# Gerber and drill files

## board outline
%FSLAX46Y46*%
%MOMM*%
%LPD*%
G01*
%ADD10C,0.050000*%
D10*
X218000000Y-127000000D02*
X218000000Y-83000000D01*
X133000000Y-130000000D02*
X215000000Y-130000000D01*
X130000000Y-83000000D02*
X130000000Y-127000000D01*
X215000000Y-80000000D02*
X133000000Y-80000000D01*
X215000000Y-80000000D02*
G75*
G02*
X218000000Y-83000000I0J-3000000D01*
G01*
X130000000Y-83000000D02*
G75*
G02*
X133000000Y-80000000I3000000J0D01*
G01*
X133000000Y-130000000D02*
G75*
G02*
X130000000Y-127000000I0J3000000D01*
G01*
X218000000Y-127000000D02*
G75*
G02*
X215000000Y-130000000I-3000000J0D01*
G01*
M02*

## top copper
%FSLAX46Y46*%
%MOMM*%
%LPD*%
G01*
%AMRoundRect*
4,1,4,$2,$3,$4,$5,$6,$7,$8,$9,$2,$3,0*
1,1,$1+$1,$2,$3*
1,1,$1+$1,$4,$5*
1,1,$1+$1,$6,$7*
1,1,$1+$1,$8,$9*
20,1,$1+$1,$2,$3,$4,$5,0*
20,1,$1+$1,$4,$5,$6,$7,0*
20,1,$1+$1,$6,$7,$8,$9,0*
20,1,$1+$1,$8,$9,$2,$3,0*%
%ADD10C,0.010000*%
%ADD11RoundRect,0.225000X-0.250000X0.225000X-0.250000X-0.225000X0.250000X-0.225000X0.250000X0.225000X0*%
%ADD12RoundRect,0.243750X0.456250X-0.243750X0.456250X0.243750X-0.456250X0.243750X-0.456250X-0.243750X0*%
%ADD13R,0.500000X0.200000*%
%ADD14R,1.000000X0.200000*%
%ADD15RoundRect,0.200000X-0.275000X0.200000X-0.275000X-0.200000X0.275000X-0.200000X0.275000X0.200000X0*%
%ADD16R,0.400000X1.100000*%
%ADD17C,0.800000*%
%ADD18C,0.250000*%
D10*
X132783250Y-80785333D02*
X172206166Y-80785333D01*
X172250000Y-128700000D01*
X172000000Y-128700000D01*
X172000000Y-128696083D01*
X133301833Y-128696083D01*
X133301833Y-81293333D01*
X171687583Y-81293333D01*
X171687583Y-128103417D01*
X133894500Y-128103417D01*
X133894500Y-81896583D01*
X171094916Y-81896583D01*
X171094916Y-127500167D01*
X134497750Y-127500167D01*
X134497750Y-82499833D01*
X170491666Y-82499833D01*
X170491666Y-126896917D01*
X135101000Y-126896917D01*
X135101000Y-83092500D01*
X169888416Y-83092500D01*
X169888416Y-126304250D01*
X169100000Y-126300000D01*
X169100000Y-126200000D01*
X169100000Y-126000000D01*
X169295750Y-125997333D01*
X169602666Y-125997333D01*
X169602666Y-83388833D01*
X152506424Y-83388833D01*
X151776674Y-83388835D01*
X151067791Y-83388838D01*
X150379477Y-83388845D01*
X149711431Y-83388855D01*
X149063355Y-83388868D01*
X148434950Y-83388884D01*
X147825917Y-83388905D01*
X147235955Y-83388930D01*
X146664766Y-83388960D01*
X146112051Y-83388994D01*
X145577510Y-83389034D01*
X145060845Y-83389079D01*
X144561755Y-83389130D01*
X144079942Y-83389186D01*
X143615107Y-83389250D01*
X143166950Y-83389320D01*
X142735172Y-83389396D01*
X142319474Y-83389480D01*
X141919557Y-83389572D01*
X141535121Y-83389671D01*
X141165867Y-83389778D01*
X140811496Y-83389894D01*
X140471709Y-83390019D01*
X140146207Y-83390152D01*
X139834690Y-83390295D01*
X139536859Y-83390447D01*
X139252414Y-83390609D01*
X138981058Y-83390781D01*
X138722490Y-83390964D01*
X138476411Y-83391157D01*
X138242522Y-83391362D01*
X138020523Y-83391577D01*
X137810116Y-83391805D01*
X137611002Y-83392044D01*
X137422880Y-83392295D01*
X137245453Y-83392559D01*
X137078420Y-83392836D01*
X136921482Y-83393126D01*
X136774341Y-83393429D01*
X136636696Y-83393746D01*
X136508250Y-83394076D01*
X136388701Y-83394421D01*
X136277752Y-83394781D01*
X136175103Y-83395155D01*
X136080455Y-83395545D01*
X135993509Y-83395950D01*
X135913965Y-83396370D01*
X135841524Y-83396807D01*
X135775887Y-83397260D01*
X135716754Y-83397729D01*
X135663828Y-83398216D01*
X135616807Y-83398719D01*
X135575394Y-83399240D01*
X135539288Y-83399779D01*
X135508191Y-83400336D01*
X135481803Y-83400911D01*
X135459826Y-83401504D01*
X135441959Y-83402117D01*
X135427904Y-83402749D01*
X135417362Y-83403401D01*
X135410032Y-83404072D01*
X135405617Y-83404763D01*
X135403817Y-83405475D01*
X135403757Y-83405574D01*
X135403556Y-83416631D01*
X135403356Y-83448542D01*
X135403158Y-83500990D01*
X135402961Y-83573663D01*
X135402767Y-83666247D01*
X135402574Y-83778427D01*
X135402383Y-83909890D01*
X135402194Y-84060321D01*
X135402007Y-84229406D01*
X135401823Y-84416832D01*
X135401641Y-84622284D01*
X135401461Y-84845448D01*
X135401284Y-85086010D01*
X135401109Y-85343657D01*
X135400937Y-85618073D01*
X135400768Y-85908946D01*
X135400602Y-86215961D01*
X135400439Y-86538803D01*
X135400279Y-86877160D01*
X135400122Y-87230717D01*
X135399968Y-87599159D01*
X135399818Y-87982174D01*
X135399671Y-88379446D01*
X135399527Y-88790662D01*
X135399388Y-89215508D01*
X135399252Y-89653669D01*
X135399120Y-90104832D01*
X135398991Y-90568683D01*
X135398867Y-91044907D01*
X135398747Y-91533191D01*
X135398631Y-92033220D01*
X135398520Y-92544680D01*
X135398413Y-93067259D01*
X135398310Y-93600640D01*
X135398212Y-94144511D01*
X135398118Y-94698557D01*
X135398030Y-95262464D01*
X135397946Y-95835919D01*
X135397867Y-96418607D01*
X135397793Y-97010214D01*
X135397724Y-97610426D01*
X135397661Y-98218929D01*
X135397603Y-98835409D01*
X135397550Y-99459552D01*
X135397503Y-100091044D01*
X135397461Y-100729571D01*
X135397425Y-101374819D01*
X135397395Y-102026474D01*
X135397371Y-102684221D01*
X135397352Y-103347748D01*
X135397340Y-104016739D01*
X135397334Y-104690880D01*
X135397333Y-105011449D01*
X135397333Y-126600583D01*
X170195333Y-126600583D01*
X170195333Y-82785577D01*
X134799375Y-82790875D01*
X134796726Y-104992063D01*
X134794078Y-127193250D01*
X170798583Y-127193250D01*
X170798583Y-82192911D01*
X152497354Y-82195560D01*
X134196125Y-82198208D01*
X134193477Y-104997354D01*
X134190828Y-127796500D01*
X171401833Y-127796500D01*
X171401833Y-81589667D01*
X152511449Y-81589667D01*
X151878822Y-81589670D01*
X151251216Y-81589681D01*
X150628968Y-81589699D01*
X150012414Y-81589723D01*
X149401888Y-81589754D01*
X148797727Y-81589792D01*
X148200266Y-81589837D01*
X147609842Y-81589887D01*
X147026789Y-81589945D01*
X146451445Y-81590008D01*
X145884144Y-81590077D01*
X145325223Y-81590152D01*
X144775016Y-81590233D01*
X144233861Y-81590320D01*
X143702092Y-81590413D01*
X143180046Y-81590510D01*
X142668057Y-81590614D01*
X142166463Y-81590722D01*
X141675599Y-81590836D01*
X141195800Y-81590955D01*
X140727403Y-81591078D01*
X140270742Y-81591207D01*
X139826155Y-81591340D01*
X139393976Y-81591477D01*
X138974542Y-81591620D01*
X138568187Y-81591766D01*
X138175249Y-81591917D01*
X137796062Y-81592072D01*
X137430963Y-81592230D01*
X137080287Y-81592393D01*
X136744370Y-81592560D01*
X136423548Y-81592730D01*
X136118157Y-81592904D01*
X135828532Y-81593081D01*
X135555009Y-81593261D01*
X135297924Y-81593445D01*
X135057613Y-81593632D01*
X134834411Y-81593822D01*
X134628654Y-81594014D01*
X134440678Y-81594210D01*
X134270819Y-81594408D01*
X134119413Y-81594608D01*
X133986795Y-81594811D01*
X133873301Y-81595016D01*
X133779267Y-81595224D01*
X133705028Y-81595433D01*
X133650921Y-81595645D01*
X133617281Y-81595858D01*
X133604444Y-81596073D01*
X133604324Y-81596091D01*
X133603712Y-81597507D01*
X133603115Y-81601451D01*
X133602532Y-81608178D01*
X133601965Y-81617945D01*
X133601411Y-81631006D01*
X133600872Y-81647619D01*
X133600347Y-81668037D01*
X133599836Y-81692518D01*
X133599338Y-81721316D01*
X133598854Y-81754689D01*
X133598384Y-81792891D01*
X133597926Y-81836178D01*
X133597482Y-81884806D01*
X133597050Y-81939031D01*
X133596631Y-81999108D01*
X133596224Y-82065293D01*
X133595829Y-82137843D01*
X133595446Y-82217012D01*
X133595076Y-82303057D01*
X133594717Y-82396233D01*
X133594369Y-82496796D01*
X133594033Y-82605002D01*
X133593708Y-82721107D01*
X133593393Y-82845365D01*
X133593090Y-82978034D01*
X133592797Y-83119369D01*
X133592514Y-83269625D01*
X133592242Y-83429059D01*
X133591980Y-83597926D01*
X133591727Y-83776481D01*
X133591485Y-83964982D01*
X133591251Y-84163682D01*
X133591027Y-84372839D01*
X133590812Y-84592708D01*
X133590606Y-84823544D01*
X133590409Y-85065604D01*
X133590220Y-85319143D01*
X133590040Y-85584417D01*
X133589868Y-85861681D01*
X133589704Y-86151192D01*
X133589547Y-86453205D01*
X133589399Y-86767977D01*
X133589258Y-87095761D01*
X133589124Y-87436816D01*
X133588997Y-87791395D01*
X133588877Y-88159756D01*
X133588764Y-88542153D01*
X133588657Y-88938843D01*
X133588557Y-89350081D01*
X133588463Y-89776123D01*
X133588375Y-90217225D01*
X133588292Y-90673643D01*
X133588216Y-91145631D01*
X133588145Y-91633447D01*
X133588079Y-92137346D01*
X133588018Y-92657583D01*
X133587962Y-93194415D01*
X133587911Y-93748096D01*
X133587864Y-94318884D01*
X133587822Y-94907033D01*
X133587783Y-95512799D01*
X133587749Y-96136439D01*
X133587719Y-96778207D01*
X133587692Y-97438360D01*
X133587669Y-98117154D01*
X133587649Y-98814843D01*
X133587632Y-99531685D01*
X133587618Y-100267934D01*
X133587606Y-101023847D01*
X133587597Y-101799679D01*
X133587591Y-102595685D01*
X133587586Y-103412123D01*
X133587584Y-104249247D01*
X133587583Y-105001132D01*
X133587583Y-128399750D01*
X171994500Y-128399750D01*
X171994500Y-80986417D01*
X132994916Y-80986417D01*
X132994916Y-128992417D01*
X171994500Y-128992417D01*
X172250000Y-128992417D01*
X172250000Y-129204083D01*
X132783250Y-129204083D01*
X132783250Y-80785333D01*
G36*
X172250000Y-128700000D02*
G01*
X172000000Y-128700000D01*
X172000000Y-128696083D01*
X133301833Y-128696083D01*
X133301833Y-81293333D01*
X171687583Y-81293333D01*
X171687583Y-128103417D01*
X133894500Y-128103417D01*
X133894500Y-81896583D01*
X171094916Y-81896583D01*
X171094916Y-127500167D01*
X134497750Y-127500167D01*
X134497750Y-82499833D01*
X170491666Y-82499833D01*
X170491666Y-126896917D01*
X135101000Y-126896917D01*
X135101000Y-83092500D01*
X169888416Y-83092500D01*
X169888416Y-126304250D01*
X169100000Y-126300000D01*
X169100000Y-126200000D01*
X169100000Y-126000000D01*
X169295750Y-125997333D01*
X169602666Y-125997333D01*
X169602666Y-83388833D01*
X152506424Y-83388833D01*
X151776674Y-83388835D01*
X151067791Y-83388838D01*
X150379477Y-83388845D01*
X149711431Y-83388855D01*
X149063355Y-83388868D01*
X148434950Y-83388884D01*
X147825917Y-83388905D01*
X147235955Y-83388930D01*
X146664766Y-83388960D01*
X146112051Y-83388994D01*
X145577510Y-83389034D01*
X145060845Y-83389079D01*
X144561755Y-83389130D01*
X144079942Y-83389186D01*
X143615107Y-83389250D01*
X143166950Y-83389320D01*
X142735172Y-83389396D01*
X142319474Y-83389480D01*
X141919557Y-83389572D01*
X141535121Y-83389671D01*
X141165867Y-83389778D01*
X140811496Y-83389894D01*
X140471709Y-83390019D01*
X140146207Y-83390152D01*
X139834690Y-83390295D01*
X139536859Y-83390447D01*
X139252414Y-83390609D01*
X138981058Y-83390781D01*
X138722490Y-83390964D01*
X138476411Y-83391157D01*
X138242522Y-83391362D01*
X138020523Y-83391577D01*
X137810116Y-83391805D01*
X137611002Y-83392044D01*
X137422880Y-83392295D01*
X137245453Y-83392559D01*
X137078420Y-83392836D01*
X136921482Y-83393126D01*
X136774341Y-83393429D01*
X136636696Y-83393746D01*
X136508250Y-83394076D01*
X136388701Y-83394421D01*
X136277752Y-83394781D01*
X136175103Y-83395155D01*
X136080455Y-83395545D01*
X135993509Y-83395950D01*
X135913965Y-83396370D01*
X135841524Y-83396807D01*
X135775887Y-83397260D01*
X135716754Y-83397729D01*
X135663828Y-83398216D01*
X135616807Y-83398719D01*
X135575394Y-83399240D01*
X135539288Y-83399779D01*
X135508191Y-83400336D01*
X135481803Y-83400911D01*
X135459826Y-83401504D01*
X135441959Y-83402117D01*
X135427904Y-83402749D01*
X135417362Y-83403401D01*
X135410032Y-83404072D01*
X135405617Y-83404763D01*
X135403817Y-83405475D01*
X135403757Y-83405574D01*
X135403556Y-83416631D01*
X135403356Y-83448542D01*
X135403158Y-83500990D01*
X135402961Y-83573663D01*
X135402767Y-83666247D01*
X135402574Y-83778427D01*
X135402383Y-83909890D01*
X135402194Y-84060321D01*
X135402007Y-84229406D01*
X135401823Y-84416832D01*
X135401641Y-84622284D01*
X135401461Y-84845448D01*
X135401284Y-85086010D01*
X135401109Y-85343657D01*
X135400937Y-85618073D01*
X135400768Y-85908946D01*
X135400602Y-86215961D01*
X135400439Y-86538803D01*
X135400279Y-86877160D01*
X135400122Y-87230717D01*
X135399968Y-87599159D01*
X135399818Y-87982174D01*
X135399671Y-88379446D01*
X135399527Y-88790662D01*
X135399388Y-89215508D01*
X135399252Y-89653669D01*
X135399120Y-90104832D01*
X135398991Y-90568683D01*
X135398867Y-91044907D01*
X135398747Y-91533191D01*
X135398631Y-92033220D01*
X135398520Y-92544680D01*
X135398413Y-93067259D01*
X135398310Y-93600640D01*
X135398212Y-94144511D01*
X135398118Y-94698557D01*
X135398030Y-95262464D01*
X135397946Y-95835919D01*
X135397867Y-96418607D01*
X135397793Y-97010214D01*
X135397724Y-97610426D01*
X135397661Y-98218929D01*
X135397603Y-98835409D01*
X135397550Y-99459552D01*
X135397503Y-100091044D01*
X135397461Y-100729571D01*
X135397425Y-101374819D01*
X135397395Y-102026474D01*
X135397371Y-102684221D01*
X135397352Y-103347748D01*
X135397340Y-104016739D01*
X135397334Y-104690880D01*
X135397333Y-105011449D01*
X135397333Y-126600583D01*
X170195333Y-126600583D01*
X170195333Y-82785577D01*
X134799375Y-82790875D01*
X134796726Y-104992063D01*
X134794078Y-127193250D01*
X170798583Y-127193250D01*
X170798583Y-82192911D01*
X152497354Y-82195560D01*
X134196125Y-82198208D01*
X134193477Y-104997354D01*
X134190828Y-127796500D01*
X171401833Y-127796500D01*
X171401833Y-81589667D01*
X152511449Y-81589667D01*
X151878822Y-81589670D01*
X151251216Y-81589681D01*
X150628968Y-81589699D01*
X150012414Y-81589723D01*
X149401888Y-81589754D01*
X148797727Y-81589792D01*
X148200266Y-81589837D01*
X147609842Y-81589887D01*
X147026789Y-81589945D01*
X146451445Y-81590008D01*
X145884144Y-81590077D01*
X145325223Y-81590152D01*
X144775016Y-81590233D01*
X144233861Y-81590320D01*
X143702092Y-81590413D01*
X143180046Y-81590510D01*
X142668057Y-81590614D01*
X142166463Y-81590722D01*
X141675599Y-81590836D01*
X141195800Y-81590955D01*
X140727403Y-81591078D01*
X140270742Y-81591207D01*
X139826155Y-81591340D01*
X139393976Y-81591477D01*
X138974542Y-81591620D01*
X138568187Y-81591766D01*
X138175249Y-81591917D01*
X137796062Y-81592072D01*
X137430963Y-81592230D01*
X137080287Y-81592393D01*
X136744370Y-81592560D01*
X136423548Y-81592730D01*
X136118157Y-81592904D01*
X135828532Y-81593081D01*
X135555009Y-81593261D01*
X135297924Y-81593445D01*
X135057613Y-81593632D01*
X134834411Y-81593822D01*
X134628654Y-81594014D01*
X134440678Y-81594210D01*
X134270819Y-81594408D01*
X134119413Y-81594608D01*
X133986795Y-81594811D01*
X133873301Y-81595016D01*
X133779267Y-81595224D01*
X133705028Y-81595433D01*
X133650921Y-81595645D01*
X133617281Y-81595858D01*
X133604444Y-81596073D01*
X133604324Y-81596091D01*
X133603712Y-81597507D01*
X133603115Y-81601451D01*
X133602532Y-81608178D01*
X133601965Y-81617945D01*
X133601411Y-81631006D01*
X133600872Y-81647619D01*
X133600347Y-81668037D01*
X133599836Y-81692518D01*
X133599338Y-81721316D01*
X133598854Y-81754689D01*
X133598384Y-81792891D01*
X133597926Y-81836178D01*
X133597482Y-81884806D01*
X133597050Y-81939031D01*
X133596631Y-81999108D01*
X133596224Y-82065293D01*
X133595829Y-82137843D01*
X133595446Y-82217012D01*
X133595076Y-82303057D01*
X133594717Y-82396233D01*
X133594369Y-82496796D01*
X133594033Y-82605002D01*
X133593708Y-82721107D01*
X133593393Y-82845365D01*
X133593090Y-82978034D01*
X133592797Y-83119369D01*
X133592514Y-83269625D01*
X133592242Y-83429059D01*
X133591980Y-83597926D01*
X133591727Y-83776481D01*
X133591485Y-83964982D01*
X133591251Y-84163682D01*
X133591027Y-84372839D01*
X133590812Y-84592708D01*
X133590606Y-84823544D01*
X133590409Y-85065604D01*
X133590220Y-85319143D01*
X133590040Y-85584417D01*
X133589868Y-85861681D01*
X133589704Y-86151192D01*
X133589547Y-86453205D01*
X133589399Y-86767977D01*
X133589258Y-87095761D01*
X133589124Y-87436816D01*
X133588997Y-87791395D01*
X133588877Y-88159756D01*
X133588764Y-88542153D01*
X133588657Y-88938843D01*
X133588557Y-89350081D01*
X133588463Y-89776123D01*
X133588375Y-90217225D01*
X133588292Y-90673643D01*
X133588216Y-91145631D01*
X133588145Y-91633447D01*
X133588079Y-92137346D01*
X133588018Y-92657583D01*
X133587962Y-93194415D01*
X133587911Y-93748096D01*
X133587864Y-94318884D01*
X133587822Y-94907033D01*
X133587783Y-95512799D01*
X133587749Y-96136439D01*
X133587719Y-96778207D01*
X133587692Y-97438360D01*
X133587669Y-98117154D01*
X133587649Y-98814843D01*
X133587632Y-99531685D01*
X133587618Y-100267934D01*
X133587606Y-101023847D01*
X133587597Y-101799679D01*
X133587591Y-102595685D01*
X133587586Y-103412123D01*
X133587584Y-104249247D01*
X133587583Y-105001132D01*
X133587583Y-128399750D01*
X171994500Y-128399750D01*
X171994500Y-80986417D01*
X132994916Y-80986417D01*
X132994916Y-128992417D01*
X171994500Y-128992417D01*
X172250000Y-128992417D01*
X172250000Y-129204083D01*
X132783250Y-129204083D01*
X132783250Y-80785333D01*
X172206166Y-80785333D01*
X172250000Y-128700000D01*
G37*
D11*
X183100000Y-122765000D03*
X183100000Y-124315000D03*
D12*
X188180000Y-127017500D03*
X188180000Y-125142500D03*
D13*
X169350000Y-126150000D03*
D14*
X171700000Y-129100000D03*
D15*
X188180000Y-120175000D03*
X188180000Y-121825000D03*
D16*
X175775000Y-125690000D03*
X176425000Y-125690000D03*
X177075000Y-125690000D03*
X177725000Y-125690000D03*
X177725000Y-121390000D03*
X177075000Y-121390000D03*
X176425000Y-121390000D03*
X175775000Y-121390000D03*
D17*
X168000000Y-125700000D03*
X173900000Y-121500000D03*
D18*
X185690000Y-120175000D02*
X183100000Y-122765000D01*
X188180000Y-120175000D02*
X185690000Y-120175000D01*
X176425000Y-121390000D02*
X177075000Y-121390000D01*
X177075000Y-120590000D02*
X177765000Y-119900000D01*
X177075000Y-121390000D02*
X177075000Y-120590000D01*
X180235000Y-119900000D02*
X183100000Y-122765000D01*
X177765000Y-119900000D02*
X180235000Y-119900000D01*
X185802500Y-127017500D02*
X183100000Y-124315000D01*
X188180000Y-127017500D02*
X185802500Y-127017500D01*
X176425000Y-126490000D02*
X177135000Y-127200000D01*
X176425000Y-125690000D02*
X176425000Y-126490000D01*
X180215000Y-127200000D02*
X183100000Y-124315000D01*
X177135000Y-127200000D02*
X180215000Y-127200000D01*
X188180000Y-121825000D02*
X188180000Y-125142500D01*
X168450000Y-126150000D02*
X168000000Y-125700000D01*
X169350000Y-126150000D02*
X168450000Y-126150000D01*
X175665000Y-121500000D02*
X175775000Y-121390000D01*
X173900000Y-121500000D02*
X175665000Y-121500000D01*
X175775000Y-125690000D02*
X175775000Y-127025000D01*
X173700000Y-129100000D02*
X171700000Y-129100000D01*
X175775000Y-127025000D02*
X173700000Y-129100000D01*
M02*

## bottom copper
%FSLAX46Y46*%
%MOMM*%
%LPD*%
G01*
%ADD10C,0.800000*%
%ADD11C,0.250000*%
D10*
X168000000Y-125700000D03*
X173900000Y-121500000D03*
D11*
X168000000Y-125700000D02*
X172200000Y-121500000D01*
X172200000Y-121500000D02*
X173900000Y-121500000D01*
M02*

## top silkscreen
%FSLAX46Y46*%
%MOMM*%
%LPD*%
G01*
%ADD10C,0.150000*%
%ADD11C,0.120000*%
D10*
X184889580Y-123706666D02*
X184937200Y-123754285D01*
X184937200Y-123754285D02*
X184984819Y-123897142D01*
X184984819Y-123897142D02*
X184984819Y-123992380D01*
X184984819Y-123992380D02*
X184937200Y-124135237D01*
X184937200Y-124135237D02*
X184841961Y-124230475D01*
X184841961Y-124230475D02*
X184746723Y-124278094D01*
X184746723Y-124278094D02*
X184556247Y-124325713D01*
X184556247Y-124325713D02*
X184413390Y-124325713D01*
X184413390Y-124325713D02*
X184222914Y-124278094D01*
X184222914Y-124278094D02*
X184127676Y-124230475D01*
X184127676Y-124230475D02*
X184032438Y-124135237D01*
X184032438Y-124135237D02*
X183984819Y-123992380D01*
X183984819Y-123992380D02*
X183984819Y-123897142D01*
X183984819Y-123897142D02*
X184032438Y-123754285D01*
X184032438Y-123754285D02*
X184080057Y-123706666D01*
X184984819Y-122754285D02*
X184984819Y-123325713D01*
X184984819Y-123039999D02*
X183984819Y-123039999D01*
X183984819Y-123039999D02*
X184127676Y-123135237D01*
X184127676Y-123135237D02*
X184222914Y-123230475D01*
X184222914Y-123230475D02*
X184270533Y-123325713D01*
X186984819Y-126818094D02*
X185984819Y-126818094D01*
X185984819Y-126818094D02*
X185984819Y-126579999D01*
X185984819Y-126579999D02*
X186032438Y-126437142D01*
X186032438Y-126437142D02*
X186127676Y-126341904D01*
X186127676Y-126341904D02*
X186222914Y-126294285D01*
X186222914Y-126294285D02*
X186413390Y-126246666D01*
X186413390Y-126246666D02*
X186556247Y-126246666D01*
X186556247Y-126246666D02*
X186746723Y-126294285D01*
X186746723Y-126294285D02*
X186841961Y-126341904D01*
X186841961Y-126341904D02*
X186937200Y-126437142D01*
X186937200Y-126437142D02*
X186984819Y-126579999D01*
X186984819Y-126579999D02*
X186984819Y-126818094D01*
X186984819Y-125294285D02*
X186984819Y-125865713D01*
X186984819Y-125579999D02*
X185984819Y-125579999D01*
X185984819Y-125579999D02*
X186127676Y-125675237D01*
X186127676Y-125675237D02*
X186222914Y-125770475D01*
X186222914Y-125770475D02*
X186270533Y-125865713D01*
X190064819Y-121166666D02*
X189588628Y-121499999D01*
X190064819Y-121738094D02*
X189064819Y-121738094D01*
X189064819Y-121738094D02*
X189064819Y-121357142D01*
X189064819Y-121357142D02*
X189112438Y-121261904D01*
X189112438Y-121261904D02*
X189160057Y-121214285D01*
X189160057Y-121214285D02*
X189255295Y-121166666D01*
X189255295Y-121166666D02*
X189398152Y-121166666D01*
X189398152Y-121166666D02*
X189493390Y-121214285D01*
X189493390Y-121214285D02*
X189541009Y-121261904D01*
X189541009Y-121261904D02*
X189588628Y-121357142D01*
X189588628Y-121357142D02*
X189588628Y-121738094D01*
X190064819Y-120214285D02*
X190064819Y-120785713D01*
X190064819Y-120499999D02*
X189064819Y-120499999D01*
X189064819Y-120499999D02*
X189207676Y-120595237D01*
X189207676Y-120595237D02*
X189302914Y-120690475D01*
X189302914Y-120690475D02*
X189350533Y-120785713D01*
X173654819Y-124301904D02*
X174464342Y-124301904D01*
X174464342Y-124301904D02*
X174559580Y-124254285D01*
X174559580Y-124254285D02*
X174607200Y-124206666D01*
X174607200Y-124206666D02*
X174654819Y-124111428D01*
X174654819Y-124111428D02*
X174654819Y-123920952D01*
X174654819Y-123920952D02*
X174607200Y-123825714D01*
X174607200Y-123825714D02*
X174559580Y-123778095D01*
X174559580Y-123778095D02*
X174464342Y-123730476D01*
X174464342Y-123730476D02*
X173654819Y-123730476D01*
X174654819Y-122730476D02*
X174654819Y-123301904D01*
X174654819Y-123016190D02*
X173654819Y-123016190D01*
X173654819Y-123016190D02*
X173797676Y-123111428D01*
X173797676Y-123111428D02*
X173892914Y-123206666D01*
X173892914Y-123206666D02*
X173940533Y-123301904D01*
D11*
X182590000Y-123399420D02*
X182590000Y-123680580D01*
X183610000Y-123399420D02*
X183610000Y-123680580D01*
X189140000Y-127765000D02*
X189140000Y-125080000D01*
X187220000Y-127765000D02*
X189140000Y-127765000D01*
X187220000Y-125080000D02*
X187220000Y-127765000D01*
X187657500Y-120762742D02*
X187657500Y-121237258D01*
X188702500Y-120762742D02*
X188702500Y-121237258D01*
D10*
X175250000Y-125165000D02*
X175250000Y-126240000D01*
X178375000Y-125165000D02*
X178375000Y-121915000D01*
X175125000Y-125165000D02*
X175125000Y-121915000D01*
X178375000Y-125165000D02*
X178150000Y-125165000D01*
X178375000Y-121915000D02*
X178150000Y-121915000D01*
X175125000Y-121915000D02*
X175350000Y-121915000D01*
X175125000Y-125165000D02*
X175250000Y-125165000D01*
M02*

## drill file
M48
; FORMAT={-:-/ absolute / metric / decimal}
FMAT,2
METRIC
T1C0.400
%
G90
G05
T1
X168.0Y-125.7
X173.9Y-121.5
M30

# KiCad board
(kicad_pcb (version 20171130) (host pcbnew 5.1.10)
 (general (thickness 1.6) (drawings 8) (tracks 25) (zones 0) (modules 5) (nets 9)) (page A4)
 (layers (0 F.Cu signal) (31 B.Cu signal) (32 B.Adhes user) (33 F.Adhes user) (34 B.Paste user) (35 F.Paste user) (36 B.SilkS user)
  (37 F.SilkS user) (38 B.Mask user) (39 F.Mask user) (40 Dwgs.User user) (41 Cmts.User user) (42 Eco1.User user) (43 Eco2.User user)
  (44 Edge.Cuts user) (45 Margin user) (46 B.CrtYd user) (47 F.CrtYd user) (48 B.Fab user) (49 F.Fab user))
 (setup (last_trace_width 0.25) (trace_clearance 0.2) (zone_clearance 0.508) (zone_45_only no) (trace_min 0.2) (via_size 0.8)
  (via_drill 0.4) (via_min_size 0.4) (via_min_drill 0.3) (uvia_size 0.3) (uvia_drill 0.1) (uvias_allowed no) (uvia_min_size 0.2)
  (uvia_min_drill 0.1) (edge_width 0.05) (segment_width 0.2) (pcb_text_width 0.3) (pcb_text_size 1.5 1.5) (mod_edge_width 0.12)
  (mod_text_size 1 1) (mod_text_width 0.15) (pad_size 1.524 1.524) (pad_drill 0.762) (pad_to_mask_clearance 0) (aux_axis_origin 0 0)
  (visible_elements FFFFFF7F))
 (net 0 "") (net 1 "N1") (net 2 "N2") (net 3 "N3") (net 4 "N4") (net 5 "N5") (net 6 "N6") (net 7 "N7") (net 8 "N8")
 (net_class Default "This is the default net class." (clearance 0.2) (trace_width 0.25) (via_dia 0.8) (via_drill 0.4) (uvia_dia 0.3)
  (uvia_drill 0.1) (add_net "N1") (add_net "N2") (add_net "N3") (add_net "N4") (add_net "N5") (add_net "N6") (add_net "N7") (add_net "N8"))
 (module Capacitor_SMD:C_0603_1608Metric (layer F.Cu) (at 183.1 123.54 270)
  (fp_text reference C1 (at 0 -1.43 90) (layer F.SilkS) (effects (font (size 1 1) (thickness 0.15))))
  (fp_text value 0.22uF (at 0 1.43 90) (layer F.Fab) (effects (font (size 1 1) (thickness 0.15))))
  (fp_line (start -0.14058 0.51) (end 0.14058 0.51) (layer F.SilkS) (width 0.12))
  (fp_line (start -0.14058 -0.51) (end 0.14058 -0.51) (layer F.SilkS) (width 0.12))
  (pad 1 smd roundrect (at -0.775 0 270) (size 0.9 0.95) (layers F.Cu F.Paste F.Mask) (roundrect_rratio 0.25) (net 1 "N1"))
  (pad 2 smd roundrect (at 0.775 0 270) (size 0.9 0.95) (layers F.Cu F.Paste F.Mask) (roundrect_rratio 0.25) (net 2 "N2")))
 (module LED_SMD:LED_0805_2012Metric (layer F.Cu) (at 188.18 126.08 90)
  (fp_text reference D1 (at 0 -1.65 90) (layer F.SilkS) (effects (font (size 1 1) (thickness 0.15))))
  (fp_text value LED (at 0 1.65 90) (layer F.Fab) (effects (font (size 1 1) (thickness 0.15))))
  (fp_line (start -1.685 0.96) (end 1 0.96) (layer F.SilkS) (width 0.12))
  (fp_line (start -1.685 -0.96) (end -1.685 0.96) (layer F.SilkS) (width 0.12))
  (fp_line (start 1 -0.96) (end -1.685 -0.96) (layer F.SilkS) (width 0.12))
  (pad 1 smd roundrect (at -0.9375 0 90) (size 0.975 1.4) (layers F.Cu F.Paste F.Mask) (roundrect_rratio 0.25) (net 2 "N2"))
  (pad 2 smd roundrect (at 0.9375 0 90) (size 0.975 1.4) (layers F.Cu F.Paste F.Mask) (roundrect_rratio 0.25) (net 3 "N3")))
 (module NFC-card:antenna (layer F.Cu) (at 152.5 105 180)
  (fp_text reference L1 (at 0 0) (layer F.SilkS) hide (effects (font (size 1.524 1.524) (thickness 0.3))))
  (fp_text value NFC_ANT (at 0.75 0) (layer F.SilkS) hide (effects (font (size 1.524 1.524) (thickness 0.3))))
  (fp_poly
   (pts (xy 19.71675 24.214667) (xy -19.706166 24.214667) (xy -19.75 -23.7) (xy -19.5 -23.7) (xy -19.5 -23.696083) (xy 19.198167 -23.696083)
    (xy 19.198167 23.706667) (xy -19.187583 23.706667) (xy -19.187583 -23.103417) (xy 18.6055 -23.103417) (xy 18.6055 23.103417)
    (xy -18.594916 23.103417) (xy -18.594916 -22.500167) (xy 18.00225 -22.500167) (xy 18.00225 22.500167) (xy -17.991666 22.500167)
    (xy -17.991666 -21.896917) (xy 17.399 -21.896917) (xy 17.399 21.9075) (xy -17.388416 21.9075) (xy -17.388416 -21.30425) (xy -16.6 -21.3)
    (xy -16.6 -21.2) (xy -16.6 -21) (xy -16.79575 -20.997333) (xy -17.102666 -20.997333) (xy -17.102666 21.611167) (xy -0.006424 21.611167)
    (xy 0.723326 21.611165) (xy 1.432209 21.611162) (xy 2.120523 21.611155) (xy 2.788569 21.611145) (xy 3.436645 21.611132)
    (xy 4.06505 21.611116) (xy 4.674083 21.611095) (xy 5.264045 21.61107) (xy 5.835234 21.61104) (xy 6.387949 21.611006)
    (xy 6.92249 21.610966) (xy 7.439155 21.610921) (xy 7.938245 21.61087) (xy 8.420058 21.610814) (xy 8.884893 21.61075)
    (xy 9.33305 21.61068) (xy 9.764828 21.610604) (xy 10.180526 21.61052) (xy 10.580443 21.610428) (xy 10.964879 21.610329)
    (xy 11.334133 21.610222) (xy 11.688504 21.610106) (xy 12.028291 21.609981) (xy 12.353793 21.609848) (xy 12.66531 21.609705)
    (xy 12.963141 21.609553) (xy 13.247586 21.609391) (xy 13.518942 21.609219) (xy 13.77751 21.609036) (xy 14.023589 21.608843)
    (xy 14.257478 21.608638) (xy 14.479477 21.608423) (xy 14.689884 21.608195) (xy 14.888998 21.607956) (xy 15.07712 21.607705)
    (xy 15.254547 21.607441) (xy 15.42158 21.607164) (xy 15.578518 21.606874) (xy 15.725659 21.606571) (xy 15.863304 21.606254)
    (xy 15.99175 21.605924) (xy 16.111299 21.605579) (xy 16.222248 21.605219) (xy 16.324897 21.604845) (xy 16.419545 21.604455)
    (xy 16.506491 21.60405) (xy 16.586035 21.60363) (xy 16.658476 21.603193) (xy 16.724113 21.60274) (xy 16.783246 21.602271)
    (xy 16.836172 21.601784) (xy 16.883193 21.601281) (xy 16.924606 21.60076) (xy 16.960712 21.600221) (xy 16.991809 21.599664)
    (xy 17.018197 21.599089) (xy 17.040174 21.598496) (xy 17.058041 21.597883) (xy 17.072096 21.597251) (xy 17.082638 21.596599)
    (xy 17.089968 21.595928) (xy 17.094383 21.595237) (xy 17.096183 21.594525) (xy 17.096243 21.594426) (xy 17.096444 21.583369)
    (xy 17.096644 21.551458) (xy 17.096842 21.49901) (xy 17.097039 21.426337) (xy 17.097233 21.333753) (xy 17.097426 21.221573)
    (xy 17.097617 21.09011) (xy 17.097806 20.939679) (xy 17.097993 20.770594) (xy 17.098177 20.583168) (xy 17.098359 20.377716)
    (xy 17.098539 20.154552) (xy 17.098716 19.91399) (xy 17.098891 19.656343) (xy 17.099063 19.381927) (xy 17.099232 19.091054)
    (xy 17.099398 18.784039) (xy 17.099561 18.461197) (xy 17.099721 18.12284) (xy 17.099878 17.769283) (xy 17.100032 17.400841)
    (xy 17.100182 17.017826) (xy 17.100329 16.620554) (xy 17.100473 16.209338) (xy 17.100612 15.784492) (xy 17.100748 15.346331)
    (xy 17.10088 14.895168) (xy 17.101009 14.431317) (xy 17.101133 13.955093) (xy 17.101253 13.466809) (xy 17.101369 12.96678)
    (xy 17.10148 12.45532) (xy 17.101587 11.932741) (xy 17.10169 11.39936) (xy 17.101788 10.855489) (xy 17.101882 10.301443)
    (xy 17.10197 9.737536) (xy 17.102054 9.164081) (xy 17.102133 8.581393) (xy 17.102207 7.989786) (xy 17.102276 7.389574)
    (xy 17.102339 6.781071) (xy 17.102397 6.164591) (xy 17.10245 5.540448) (xy 17.102497 4.908956) (xy 17.102539 4.270429)
    (xy 17.102575 3.625181) (xy 17.102605 2.973526) (xy 17.102629 2.315779) (xy 17.102648 1.652252) (xy 17.10266 0.983261)
    (xy 17.102666 0.30912) (xy 17.102667 -0.011449) (xy 17.102667 -21.600583) (xy -17.695333 -21.600583) (xy -17.695333 22.214423)
    (xy 17.700625 22.209125) (xy 17.703274 0.007937) (xy 17.705922 -22.19325) (xy -18.298583 -22.19325) (xy -18.298583 22.807089)
    (xy 0.002646 22.80444) (xy 18.303875 22.801792) (xy 18.306523 0.002646) (xy 18.309172 -22.7965) (xy -18.901833 -22.7965)
    (xy -18.901833 23.410333) (xy -0.011449 23.410333) (xy 0.621178 23.41033) (xy 1.248784 23.410319) (xy 1.871032 23.410301)
    (xy 2.487586 23.410277) (xy 3.098112 23.410246) (xy 3.702273 23.410208) (xy 4.299734 23.410163) (xy 4.890158 23.410113)
    (xy 5.473211 23.410055) (xy 6.048555 23.409992) (xy 6.615856 23.409923) (xy 7.174777 23.409848) (xy 7.724984 23.409767)
    (xy 8.266139 23.40968) (xy 8.797908 23.409587) (xy 9.319954 23.40949) (xy 9.831943 23.409386) (xy 10.333537 23.409278)
    (xy 10.824401 23.409164) (xy 11.3042 23.409045) (xy 11.772597 23.408922) (xy 12.229258 23.408793) (xy 12.673845 23.40866)
    (xy 13.106024 23.408523) (xy 13.525458 23.40838) (xy 13.931813 23.408234) (xy 14.324751 23.408083) (xy 14.703938 23.407928)
    (xy 15.069037 23.40777) (xy 15.419713 23.407607) (xy 15.75563 23.40744) (xy 16.076452 23.40727) (xy 16.381843 23.407096)
    (xy 16.671468 23.406919) (xy 16.944991 23.406739) (xy 17.202076 23.406555) (xy 17.442387 23.406368) (xy 17.665589 23.406178)
    (xy 17.871346 23.405986) (xy 18.059322 23.40579) (xy 18.229181 23.405592) (xy 18.380587 23.405392) (xy 18.513205 23.405189)
    (xy 18.626699 23.404984) (xy 18.720733 23.404776) (xy 18.794972 23.404567) (xy 18.849079 23.404355) (xy 18.882719 23.404142)
    (xy 18.895556 23.403927) (xy 18.895676 23.403909) (xy 18.896288 23.402493) (xy 18.896885 23.398549) (xy 18.897468 23.391822)
    (xy 18.898035 23.382055) (xy 18.898589 23.368994) (xy 18.899128 23.352381) (xy 18.899653 23.331963) (xy 18.900164 23.307482)
    (xy 18.900662 23.278684) (xy 18.901146 23.245311) (xy 18.901616 23.207109) (xy 18.902074 23.163822) (xy 18.902518 23.115194)
    (xy 18.90295 23.060969) (xy 18.903369 23.000892) (xy 18.903776 22.934707) (xy 18.904171 22.862157) (xy 18.904554 22.782988)
    (xy 18.904924 22.696943) (xy 18.905283 22.603767) (xy 18.905631 22.503204) (xy 18.905967 22.394998) (xy 18.906292 22.278893)
    (xy 18.906607 22.154635) (xy 18.90691 22.021966) (xy 18.907203 21.880631) (xy 18.907486 21.730375) (xy 18.907758 21.570941)
    (xy 18.90802 21.402074) (xy 18.908273 21.223519) (xy 18.908515 21.035018) (xy 18.908749 20.836318) (xy 18.908973 20.627161)
    (xy 18.909188 20.407292) (xy 18.909394 20.176456) (xy 18.909591 19.934396) (xy 18.90978 19.680857) (xy 18.90996 19.415583)
    (xy 18.910132 19.138319) (xy 18.910296 18.848808) (xy 18.910453 18.546795) (xy 18.910601 18.232023) (xy 18.910742 17.904239)
    (xy 18.910876 17.563184) (xy 18.911003 17.208605) (xy 18.911123 16.840244) (xy 18.911236 16.457847) (xy 18.911343 16.061157)
    (xy 18.911443 15.649919) (xy 18.911537 15.223877) (xy 18.911625 14.782775) (xy 18.911708 14.326357) (xy 18.911784 13.854369)
    (xy 18.911855 13.366553) (xy 18.911921 12.862654) (xy 18.911982 12.342417) (xy 18.912038 11.805585) (xy 18.912089 11.251904)
    (xy 18.912136 10.681116) (xy 18.912178 10.092967) (xy 18.912217 9.487201) (xy 18.912251 8.863561) (xy 18.912281 8.221793)
    (xy 18.912308 7.56164) (xy 18.912331 6.882846) (xy 18.912351 6.185157) (xy 18.912368 5.468315) (xy 18.912382 4.732066)
    (xy 18.912394 3.976153) (xy 18.912403 3.200321) (xy 18.912409 2.404315) (xy 18.912414 1.587877) (xy 18.912416 0.750753)
    (xy 18.912417 -0.001132) (xy 18.912417 -23.39975) (xy -19.4945 -23.39975) (xy -19.4945 24.013583) (xy 19.505084 24.013583)
    (xy 19.505084 -23.992417) (xy -19.4945 -23.992417) (xy -19.75 -23.992417) (xy -19.75 -24.204083) (xy 19.71675 -24.204083)
    (xy 19.71675 24.214667))
   (layer F.Cu) (width 0.01))
  (pad 1 smd rect (at -16.85 -21.15 180) (size 0.5 0.2) (layers F.Cu F.Paste) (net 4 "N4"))
  (pad 2 smd rect (at -19.2 -24.1 180) (size 1 0.2) (layers F.Cu F.Paste) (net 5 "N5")))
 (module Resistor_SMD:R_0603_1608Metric (layer F.Cu) (at 188.18 121 270)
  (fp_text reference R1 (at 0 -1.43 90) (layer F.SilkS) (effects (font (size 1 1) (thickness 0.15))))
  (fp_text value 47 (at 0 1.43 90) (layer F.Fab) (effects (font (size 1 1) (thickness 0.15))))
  (fp_line (start -0.237258 0.5225) (end 0.237258 0.5225) (layer F.SilkS) (width 0.12))
  (fp_line (start -0.237258 -0.5225) (end 0.237258 -0.5225) (layer F.SilkS) (width 0.12))
  (pad 1 smd roundrect (at -0.825 0 270) (size 0.8 0.95) (layers F.Cu F.Paste F.Mask) (roundrect_rratio 0.25) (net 1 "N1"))
  (pad 2 smd roundrect (at 0.825 0 270) (size 0.8 0.95) (layers F.Cu F.Paste F.Mask) (roundrect_rratio 0.25) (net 3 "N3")))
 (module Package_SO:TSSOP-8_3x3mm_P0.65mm (layer F.Cu) (at 176.75 123.54 90)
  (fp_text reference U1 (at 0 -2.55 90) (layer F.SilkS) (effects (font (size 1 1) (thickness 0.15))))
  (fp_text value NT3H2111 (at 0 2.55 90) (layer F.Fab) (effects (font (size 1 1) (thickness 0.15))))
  (fp_line (start -1.625 -1.5) (end -2.7 -1.5) (layer F.SilkS) (width 0.15))
  (fp_line (start -1.625 1.625) (end 1.625 1.625) (layer F.SilkS) (width 0.15))
  (fp_line (start -1.625 -1.625) (end 1.625 -1.625) (layer F.SilkS) (width 0.15))
  (fp_line (start -1.625 1.625) (end -1.625 1.4) (layer F.SilkS) (width 0.15))
  (fp_line (start 1.625 1.625) (end 1.625 1.4) (layer F.SilkS) (width 0.15))
  (fp_line (start 1.625 -1.625) (end 1.625 -1.4) (layer F.SilkS) (width 0.15))
  (fp_line (start -1.625 -1.625) (end -1.625 -1.5) (layer F.SilkS) (width 0.15))
  (pad 1 smd rect (at -2.15 -0.975 90) (size 1.1 0.4) (layers F.Cu F.Paste F.Mask) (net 5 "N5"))
  (pad 2 smd rect (at -2.15 -0.325 90) (size 1.1 0.4) (layers F.Cu F.Paste F.Mask) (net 2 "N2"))
  (pad 3 smd rect (at -2.15 0.325 90) (size 1.1 0.4) (layers F.Cu F.Paste F.Mask) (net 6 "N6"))
  (pad 4 smd rect (at -2.15 0.975 90) (size 1.1 0.4) (layers F.Cu F.Paste F.Mask) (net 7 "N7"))
  (pad 5 smd rect (at 2.15 0.975 90) (size 1.1 0.4) (layers F.Cu F.Paste F.Mask) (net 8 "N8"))
  (pad 6 smd rect (at 2.15 0.325 90) (size 1.1 0.4) (layers F.Cu F.Paste F.Mask) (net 1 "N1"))
  (pad 7 smd rect (at 2.15 -0.325 90) (size 1.1 0.4) (layers F.Cu F.Paste F.Mask) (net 1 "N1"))
  (pad 8 smd rect (at 2.15 -0.975 90) (size 1.1 0.4) (layers F.Cu F.Paste F.Mask) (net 4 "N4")))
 (gr_line (start 218 127) (end 218 83) (layer Edge.Cuts) (width 0.05))
 (gr_line (start 133 130) (end 215 130) (layer Edge.Cuts) (width 0.05))
 (gr_line (start 130 83) (end 130 127) (layer Edge.Cuts) (width 0.05))
 (gr_line (start 215 80) (end 133 80) (layer Edge.Cuts) (width 0.05))
 (gr_arc (start 215 83) (end 218 83) (angle -90) (layer Edge.Cuts) (width 0.05))
 (gr_arc (start 133 83) (end 133 80) (angle -90) (layer Edge.Cuts) (width 0.05))
 (gr_arc (start 133 127) (end 130 127) (angle -90) (layer Edge.Cuts) (width 0.05))
 (gr_arc (start 215 127) (end 215 130) (angle -90) (layer Edge.Cuts) (width 0.05))
 (segment (start 185.69 120.175) (end 183.1 122.765) (width 0.25) (layer F.Cu) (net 1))
 (segment (start 188.18 120.175) (end 185.69 120.175) (width 0.25) (layer F.Cu) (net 1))
 (segment (start 176.425 121.39) (end 177.075 121.39) (width 0.25) (layer F.Cu) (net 1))
 (segment (start 177.075 120.59) (end 177.765 119.9) (width 0.25) (layer F.Cu) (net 1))
 (segment (start 177.075 121.39) (end 177.075 120.59) (width 0.25) (layer F.Cu) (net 1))
 (segment (start 180.235 119.9) (end 183.1 122.765) (width 0.25) (layer F.Cu) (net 1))
 (segment (start 177.765 119.9) (end 180.235 119.9) (width 0.25) (layer F.Cu) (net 1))
 (segment (start 185.8025 127.0175) (end 183.1 124.315) (width 0.25) (layer F.Cu) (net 2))
 (segment (start 188.18 127.0175) (end 185.8025 127.0175) (width 0.25) (layer F.Cu) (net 2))
 (segment (start 176.425 126.49) (end 177.135 127.2) (width 0.25) (layer F.Cu) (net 2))
 (segment (start 176.425 125.69) (end 176.425 126.49) (width 0.25) (layer F.Cu) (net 2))
 (segment (start 180.215 127.2) (end 183.1 124.315) (width 0.25) (layer F.Cu) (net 2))
 (segment (start 177.135 127.2) (end 180.215 127.2) (width 0.25) (layer F.Cu) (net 2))
 (segment (start 188.18 121.825) (end 188.18 125.1425) (width 0.25) (layer F.Cu) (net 3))
 (via (at 168 125.7) (size 0.8) (drill 0.4) (layers F.Cu B.Cu) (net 4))
 (segment (start 168.45 126.15) (end 168 125.7) (width 0.25) (layer F.Cu) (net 4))
 (segment (start 169.35 126.15) (end 168.45 126.15) (width 0.25) (layer F.Cu) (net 4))
 (segment (start 168 125.7) (end 172.2 121.5) (width 0.25) (layer B.Cu) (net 4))
 (via (at 173.9 121.5) (size 0.8) (drill 0.4) (layers F.Cu B.Cu) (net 4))
 (segment (start 172.2 121.5) (end 173.9 121.5) (width 0.25) (layer B.Cu) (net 4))
 (segment (start 175.665 121.5) (end 175.775 121.39) (width 0.25) (layer F.Cu) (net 4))
 (segment (start 173.9 121.5) (end 175.665 121.5) (width 0.25) (layer F.Cu) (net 4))
 (segment (start 175.775 125.69) (end 175.775 127.025) (width 0.25) (layer F.Cu) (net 5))
 (segment (start 173.7 129.1) (end 171.7 129.1) (width 0.25) (layer F.Cu) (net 5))
 (segment (start 175.775 127.025) (end 173.7 129.1) (width 0.25) (layer F.Cu) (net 5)))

